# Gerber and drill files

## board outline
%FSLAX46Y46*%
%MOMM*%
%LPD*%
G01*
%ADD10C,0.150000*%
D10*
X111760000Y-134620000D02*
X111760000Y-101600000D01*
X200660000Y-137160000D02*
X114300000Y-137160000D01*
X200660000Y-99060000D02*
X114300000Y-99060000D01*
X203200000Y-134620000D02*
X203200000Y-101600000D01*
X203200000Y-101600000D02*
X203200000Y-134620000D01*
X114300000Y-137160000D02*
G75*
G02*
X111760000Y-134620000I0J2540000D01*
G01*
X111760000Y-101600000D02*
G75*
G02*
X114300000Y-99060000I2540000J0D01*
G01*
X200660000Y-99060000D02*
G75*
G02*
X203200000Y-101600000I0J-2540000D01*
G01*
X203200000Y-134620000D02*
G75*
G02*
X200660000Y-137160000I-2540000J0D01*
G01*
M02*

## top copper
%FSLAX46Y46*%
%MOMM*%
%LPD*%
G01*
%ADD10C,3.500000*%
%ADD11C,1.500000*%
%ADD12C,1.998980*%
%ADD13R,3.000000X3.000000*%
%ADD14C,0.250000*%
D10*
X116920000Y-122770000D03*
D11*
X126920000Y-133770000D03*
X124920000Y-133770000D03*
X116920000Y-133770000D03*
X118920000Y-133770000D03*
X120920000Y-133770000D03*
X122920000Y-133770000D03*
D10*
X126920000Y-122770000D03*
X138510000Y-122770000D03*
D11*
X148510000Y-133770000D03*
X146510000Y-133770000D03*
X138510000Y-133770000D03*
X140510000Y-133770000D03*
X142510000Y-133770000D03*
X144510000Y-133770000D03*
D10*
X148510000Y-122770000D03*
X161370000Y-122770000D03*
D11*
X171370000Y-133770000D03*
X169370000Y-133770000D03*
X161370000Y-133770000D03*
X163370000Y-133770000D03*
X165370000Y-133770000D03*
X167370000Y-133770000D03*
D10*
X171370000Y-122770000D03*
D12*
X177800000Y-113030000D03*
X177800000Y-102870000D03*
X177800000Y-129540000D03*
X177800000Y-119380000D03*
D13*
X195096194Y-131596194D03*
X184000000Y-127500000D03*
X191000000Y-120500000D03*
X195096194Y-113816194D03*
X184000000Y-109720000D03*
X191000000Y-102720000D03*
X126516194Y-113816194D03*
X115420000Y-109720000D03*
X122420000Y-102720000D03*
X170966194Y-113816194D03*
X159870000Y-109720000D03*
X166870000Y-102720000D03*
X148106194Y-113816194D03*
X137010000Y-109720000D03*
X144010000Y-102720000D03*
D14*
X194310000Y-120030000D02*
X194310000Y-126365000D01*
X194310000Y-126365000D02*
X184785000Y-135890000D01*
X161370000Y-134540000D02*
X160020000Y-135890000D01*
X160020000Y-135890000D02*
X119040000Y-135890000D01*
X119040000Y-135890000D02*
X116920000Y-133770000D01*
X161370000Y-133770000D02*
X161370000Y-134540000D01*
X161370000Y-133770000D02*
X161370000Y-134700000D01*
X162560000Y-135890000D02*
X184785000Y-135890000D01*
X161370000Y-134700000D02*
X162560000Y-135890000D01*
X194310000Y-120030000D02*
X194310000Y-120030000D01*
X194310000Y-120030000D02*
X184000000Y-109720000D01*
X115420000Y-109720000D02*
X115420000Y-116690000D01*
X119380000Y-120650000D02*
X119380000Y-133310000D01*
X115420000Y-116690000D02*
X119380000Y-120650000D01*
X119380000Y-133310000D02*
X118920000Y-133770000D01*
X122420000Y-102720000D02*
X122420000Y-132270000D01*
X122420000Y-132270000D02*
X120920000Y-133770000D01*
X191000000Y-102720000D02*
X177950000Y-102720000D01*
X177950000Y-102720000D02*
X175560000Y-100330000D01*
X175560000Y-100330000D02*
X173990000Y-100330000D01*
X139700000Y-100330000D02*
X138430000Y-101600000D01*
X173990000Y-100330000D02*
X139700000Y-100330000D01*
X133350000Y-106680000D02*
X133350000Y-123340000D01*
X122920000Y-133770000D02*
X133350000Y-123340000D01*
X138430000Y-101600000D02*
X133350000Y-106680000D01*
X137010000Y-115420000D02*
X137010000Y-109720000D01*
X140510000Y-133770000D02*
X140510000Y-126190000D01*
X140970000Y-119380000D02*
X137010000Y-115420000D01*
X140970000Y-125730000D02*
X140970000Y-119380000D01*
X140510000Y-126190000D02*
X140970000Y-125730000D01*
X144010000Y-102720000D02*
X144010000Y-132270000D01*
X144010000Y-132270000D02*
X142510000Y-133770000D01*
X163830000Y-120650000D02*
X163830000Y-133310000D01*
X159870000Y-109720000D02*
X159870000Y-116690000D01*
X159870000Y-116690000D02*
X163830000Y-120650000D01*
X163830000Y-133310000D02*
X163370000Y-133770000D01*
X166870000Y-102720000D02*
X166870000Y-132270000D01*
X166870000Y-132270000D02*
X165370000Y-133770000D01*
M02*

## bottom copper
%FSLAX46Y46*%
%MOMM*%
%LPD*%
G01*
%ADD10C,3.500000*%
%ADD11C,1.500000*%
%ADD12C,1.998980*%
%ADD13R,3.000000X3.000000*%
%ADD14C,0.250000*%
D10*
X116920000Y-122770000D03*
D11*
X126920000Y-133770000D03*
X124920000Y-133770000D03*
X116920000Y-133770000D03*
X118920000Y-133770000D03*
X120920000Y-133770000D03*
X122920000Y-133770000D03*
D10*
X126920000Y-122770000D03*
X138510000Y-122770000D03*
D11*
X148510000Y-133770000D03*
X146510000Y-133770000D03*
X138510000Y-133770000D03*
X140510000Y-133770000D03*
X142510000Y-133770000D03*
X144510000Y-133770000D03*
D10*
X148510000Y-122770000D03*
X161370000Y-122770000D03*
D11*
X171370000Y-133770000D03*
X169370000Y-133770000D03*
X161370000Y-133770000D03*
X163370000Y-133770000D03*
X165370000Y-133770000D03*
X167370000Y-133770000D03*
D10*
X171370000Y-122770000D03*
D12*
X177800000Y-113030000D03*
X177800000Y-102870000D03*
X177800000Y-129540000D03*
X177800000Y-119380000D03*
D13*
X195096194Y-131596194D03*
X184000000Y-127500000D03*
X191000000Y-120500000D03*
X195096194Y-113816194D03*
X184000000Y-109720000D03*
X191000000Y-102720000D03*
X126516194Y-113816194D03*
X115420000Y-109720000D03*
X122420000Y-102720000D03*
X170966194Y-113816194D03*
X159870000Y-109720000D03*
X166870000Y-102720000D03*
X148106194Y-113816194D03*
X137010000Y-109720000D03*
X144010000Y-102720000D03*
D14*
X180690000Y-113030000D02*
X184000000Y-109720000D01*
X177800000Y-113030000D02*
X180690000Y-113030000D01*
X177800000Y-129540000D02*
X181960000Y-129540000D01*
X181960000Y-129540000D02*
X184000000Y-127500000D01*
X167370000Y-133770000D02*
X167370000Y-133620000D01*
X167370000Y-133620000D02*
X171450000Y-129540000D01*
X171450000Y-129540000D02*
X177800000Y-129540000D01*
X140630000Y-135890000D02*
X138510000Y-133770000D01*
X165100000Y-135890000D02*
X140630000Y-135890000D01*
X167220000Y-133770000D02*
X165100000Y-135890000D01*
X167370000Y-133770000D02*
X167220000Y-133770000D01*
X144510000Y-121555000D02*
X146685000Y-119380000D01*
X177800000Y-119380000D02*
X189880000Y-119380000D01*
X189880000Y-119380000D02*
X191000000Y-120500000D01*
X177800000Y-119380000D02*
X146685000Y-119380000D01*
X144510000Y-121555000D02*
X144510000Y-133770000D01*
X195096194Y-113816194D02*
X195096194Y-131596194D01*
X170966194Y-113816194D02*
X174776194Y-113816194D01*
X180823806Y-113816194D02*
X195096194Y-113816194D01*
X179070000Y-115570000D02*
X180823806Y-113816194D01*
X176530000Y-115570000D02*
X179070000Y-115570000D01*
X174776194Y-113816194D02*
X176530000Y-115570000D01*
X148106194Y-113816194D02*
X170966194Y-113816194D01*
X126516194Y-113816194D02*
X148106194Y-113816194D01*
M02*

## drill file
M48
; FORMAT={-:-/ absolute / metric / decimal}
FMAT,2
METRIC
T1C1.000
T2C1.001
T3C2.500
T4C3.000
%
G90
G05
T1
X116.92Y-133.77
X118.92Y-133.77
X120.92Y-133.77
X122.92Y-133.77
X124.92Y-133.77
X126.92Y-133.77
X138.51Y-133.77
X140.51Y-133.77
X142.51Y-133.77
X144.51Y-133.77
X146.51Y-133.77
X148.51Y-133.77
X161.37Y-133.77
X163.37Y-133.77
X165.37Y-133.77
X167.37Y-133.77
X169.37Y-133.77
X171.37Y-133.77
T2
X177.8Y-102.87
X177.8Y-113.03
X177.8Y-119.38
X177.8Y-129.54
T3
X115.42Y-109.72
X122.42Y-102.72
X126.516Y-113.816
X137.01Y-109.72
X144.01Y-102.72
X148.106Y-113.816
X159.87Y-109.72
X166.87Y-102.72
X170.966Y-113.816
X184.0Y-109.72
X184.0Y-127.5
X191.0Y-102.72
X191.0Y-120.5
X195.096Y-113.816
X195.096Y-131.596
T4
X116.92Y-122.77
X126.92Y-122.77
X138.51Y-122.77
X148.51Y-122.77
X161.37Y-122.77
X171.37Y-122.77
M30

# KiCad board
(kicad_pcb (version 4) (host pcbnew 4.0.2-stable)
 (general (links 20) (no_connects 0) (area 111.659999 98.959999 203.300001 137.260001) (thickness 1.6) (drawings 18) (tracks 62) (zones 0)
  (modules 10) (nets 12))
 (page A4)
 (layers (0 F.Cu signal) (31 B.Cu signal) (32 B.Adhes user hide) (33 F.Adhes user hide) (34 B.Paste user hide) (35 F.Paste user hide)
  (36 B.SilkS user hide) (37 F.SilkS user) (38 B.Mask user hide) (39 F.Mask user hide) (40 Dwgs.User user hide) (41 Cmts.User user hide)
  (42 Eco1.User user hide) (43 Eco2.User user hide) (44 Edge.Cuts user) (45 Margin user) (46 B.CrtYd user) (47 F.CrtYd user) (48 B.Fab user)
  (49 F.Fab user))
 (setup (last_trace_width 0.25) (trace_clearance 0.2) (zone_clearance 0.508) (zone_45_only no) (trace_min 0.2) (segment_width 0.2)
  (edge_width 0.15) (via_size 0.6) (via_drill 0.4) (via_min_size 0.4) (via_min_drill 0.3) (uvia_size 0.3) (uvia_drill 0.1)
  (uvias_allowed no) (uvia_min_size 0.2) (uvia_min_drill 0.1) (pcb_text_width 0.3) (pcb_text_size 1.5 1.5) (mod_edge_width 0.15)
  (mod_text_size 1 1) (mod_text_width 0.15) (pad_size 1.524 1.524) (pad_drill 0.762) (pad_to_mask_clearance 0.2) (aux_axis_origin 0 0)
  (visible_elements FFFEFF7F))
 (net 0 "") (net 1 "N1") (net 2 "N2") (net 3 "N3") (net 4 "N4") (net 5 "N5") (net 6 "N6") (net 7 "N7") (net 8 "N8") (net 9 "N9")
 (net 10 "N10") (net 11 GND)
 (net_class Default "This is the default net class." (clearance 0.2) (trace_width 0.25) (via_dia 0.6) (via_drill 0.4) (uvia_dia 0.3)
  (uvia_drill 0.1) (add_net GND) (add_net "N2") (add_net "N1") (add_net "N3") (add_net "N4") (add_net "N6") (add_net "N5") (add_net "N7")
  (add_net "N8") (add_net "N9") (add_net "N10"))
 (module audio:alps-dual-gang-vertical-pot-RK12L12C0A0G (layer F.Cu) (at 121.92 128.27)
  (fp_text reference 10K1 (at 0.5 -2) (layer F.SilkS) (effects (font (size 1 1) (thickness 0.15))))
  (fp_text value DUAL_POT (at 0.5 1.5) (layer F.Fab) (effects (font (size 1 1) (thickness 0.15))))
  (pad b thru_hole circle (at -5 -5.5) (size 3.5 3.5) (drill 3) (layers *.Cu *.Mask F.SilkS))
  (pad 3 thru_hole circle (at 5 5.5) (size 1.5 1.5) (drill 1) (layers *.Cu *.Mask F.SilkS))
  (pad 6 thru_hole circle (at 3 5.5) (size 1.5 1.5) (drill 1) (layers *.Cu *.Mask F.SilkS))
  (pad 2 thru_hole circle (at -5 5.5) (size 1.5 1.5) (drill 1) (layers *.Cu *.Mask F.SilkS) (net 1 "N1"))
  (pad 1 thru_hole circle (at -3 5.5) (size 1.5 1.5) (drill 1) (layers *.Cu *.Mask F.SilkS) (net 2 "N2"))
  (pad 4 thru_hole circle (at -1 5.5) (size 1.5 1.5) (drill 1) (layers *.Cu *.Mask F.SilkS) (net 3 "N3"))
  (pad 5 thru_hole circle (at 1 5.5) (size 1.5 1.5) (drill 1) (layers *.Cu *.Mask F.SilkS) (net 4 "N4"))
  (pad a thru_hole circle (at 5 -5.5) (size 3.5 3.5) (drill 3) (layers *.Cu *.Mask F.SilkS)))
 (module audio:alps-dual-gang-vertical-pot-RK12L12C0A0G (layer F.Cu) (at 143.51 128.27)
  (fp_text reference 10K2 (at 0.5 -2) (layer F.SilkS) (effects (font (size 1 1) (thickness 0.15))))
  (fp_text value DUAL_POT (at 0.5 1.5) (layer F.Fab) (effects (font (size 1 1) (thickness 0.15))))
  (pad b thru_hole circle (at -5 -5.5) (size 3.5 3.5) (drill 3) (layers *.Cu *.Mask F.SilkS))
  (pad 3 thru_hole circle (at 5 5.5) (size 1.5 1.5) (drill 1) (layers *.Cu *.Mask F.SilkS))
  (pad 6 thru_hole circle (at 3 5.5) (size 1.5 1.5) (drill 1) (layers *.Cu *.Mask F.SilkS))
  (pad 2 thru_hole circle (at -5 5.5) (size 1.5 1.5) (drill 1) (layers *.Cu *.Mask F.SilkS) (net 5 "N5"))
  (pad 1 thru_hole circle (at -3 5.5) (size 1.5 1.5) (drill 1) (layers *.Cu *.Mask F.SilkS) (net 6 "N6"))
  (pad 4 thru_hole circle (at -1 5.5) (size 1.5 1.5) (drill 1) (layers *.Cu *.Mask F.SilkS) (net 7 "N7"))
  (pad 5 thru_hole circle (at 1 5.5) (size 1.5 1.5) (drill 1) (layers *.Cu *.Mask F.SilkS) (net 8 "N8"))
  (pad a thru_hole circle (at 5 -5.5) (size 3.5 3.5) (drill 3) (layers *.Cu *.Mask F.SilkS)))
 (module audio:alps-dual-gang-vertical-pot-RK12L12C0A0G (layer F.Cu) (at 166.37 128.27)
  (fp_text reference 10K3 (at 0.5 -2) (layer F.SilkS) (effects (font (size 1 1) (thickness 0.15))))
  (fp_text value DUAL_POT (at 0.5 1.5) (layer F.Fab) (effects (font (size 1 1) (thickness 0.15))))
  (pad b thru_hole circle (at -5 -5.5) (size 3.5 3.5) (drill 3) (layers *.Cu *.Mask F.SilkS))
  (pad 3 thru_hole circle (at 5 5.5) (size 1.5 1.5) (drill 1) (layers *.Cu *.Mask F.SilkS))
  (pad 6 thru_hole circle (at 3 5.5) (size 1.5 1.5) (drill 1) (layers *.Cu *.Mask F.SilkS))
  (pad 2 thru_hole circle (at -5 5.5) (size 1.5 1.5) (drill 1) (layers *.Cu *.Mask F.SilkS) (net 1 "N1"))
  (pad 1 thru_hole circle (at -3 5.5) (size 1.5 1.5) (drill 1) (layers *.Cu *.Mask F.SilkS) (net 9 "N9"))
  (pad 4 thru_hole circle (at -1 5.5) (size 1.5 1.5) (drill 1) (layers *.Cu *.Mask F.SilkS) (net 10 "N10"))
  (pad 5 thru_hole circle (at 1 5.5) (size 1.5 1.5) (drill 1) (layers *.Cu *.Mask F.SilkS) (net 5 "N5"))
  (pad a thru_hole circle (at 5 -5.5) (size 3.5 3.5) (drill 3) (layers *.Cu *.Mask F.SilkS)))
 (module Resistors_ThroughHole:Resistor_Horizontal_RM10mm (layer F.Cu) (at 177.8 113.03 90)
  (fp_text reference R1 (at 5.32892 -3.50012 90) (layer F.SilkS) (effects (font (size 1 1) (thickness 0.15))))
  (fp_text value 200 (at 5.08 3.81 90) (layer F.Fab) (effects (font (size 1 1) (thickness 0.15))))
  (pad 1 thru_hole circle (at 0 0 90) (size 1.99898 1.99898) (drill 1.00076) (layers *.Cu *.SilkS *.Mask) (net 1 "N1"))
  (pad 2 thru_hole circle (at 10.16 0 90) (size 1.99898 1.99898) (drill 1.00076) (layers *.Cu *.SilkS *.Mask) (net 4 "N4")))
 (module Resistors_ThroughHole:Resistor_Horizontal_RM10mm (layer F.Cu) (at 177.8 129.54 90)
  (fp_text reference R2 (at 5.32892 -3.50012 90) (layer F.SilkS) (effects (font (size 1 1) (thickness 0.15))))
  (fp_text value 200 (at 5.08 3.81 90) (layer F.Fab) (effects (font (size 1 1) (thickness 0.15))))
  (pad 1 thru_hole circle (at 0 0 90) (size 1.99898 1.99898) (drill 1.00076) (layers *.Cu *.SilkS *.Mask) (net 5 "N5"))
  (pad 2 thru_hole circle (at 10.16 0 90) (size 1.99898 1.99898) (drill 1.00076) (layers *.Cu *.SilkS *.Mask) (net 8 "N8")))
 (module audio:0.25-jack (layer F.Cu) (at 190.5 127)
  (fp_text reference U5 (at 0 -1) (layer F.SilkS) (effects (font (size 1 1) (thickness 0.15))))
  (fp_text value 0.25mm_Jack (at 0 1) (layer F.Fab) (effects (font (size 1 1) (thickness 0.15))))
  (pad 3 thru_hole rect (at 4.596194 4.596194) (size 3 3) (drill oval 2.5) (layers *.Cu *.Mask F.SilkS) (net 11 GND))
  (pad 1 thru_hole rect (at -6.5 0.5) (size 3 3) (drill oval 2.5) (layers *.Cu *.Mask F.SilkS) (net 5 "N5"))
  (pad 2 thru_hole rect (at 0.5 -6.5 90) (size 3 3) (drill oval 2.5) (layers *.Cu *.Mask F.SilkS) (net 8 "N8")))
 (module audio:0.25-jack (layer F.Cu) (at 190.5 109.22)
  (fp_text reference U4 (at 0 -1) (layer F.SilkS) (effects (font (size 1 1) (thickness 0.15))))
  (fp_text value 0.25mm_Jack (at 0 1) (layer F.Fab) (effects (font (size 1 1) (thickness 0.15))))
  (pad 3 thru_hole rect (at 4.596194 4.596194) (size 3 3) (drill oval 2.5) (layers *.Cu *.Mask F.SilkS) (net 11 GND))
  (pad 1 thru_hole rect (at -6.5 0.5) (size 3 3) (drill oval 2.5) (layers *.Cu *.Mask F.SilkS) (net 1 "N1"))
  (pad 2 thru_hole rect (at 0.5 -6.5 90) (size 3 3) (drill oval 2.5) (layers *.Cu *.Mask F.SilkS) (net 4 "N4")))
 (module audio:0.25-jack (layer F.Cu) (at 121.92 109.22)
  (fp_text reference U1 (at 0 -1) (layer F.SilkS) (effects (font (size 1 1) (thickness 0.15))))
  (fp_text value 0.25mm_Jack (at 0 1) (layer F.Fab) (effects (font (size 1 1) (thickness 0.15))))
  (pad 3 thru_hole rect (at 4.596194 4.596194) (size 3 3) (drill oval 2.5) (layers *.Cu *.Mask F.SilkS) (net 11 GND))
  (pad 1 thru_hole rect (at -6.5 0.5) (size 3 3) (drill oval 2.5) (layers *.Cu *.Mask F.SilkS) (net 2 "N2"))
  (pad 2 thru_hole rect (at 0.5 -6.5 90) (size 3 3) (drill oval 2.5) (layers *.Cu *.Mask F.SilkS) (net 3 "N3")))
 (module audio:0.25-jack (layer F.Cu) (at 166.37 109.22)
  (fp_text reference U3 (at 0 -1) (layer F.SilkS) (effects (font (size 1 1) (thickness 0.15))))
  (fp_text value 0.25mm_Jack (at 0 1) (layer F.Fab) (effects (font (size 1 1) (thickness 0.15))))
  (pad 3 thru_hole rect (at 4.596194 4.596194) (size 3 3) (drill oval 2.5) (layers *.Cu *.Mask F.SilkS) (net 11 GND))
  (pad 1 thru_hole rect (at -6.5 0.5) (size 3 3) (drill oval 2.5) (layers *.Cu *.Mask F.SilkS) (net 9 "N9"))
  (pad 2 thru_hole rect (at 0.5 -6.5 90) (size 3 3) (drill oval 2.5) (layers *.Cu *.Mask F.SilkS) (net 10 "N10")))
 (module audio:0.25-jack (layer F.Cu) (at 143.51 109.22)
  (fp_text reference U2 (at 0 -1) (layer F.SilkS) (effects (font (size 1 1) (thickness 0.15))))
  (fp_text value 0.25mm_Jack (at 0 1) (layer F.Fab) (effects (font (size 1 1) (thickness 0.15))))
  (pad 3 thru_hole rect (at 4.596194 4.596194) (size 3 3) (drill oval 2.5) (layers *.Cu *.Mask F.SilkS) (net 11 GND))
  (pad 1 thru_hole rect (at -6.5 0.5) (size 3 3) (drill oval 2.5) (layers *.Cu *.Mask F.SilkS) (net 6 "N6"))
  (pad 2 thru_hole rect (at 0.5 -6.5 90) (size 3 3) (drill oval 2.5) (layers *.Cu *.Mask F.SilkS) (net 7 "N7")))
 (gr_line (start 111.76 134.62) (end 111.76 101.6) (angle 90) (layer Edge.Cuts) (width 0.15))
 (gr_line (start 200.66 137.16) (end 114.3 137.16) (angle 90) (layer Edge.Cuts) (width 0.15))
 (gr_line (start 200.66 99.06) (end 114.3 99.06) (angle 90) (layer Edge.Cuts) (width 0.15))
 (gr_line (start 203.2 134.62) (end 203.2 101.6) (angle 90) (layer Edge.Cuts) (width 0.15))
 (gr_line (start 203.2 101.6) (end 203.2 134.62) (angle 90) (layer Edge.Cuts) (width 0.15))
 (gr_arc (start 114.3 134.62) (end 114.3 137.16) (angle 90) (layer Edge.Cuts) (width 0.15))
 (gr_arc (start 114.3 101.6) (end 111.76 101.6) (angle 90) (layer Edge.Cuts) (width 0.15))
 (gr_arc (start 200.66 101.6) (end 200.66 99.06) (angle 90) (layer Edge.Cuts) (width 0.15))
 (gr_arc (start 200.66 134.62) (end 203.2 134.62) (angle 90) (layer Edge.Cuts) (width 0.15))
 (segment (start 194.31 120.03) (end 194.31 126.365) (width 0.25) (layer F.Cu) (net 1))
 (segment (start 194.31 126.365) (end 184.785 135.89) (width 0.25) (layer F.Cu) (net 1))
 (segment (start 161.37 134.54) (end 160.02 135.89) (width 0.25) (layer F.Cu) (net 1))
 (segment (start 160.02 135.89) (end 119.04 135.89) (width 0.25) (layer F.Cu) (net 1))
 (segment (start 119.04 135.89) (end 116.92 133.77) (width 0.25) (layer F.Cu) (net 1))
 (segment (start 161.37 133.77) (end 161.37 134.54) (width 0.25) (layer F.Cu) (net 1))
 (segment (start 161.37 133.77) (end 161.37 134.7) (width 0.25) (layer F.Cu) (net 1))
 (segment (start 162.56 135.89) (end 184.785 135.89) (width 0.25) (layer F.Cu) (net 1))
 (segment (start 161.37 134.7) (end 162.56 135.89) (width 0.25) (layer F.Cu) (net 1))
 (segment (start 194.31 120.03) (end 194.31 120.03) (width 0.25) (layer F.Cu) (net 1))
 (segment (start 194.31 120.03) (end 184 109.72) (width 0.25) (layer F.Cu) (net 1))
 (segment (start 180.69 113.03) (end 184 109.72) (width 0.25) (layer B.Cu) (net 1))
 (segment (start 177.8 113.03) (end 180.69 113.03) (width 0.25) (layer B.Cu) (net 1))
 (segment (start 115.42 109.72) (end 115.42 116.69) (width 0.25) (layer F.Cu) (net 2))
 (segment (start 119.38 120.65) (end 119.38 133.31) (width 0.25) (layer F.Cu) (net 2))
 (segment (start 115.42 116.69) (end 119.38 120.65) (width 0.25) (layer F.Cu) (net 2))
 (segment (start 119.38 133.31) (end 118.92 133.77) (width 0.25) (layer F.Cu) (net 2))
 (segment (start 122.42 102.72) (end 122.42 132.27) (width 0.25) (layer F.Cu) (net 3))
 (segment (start 122.42 132.27) (end 120.92 133.77) (width 0.25) (layer F.Cu) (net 3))
 (segment (start 191 102.72) (end 177.95 102.72) (width 0.25) (layer F.Cu) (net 4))
 (segment (start 177.95 102.72) (end 175.56 100.33) (width 0.25) (layer F.Cu) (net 4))
 (segment (start 175.56 100.33) (end 173.99 100.33) (width 0.25) (layer F.Cu) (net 4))
 (segment (start 139.7 100.33) (end 138.43 101.6) (width 0.25) (layer F.Cu) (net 4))
 (segment (start 173.99 100.33) (end 139.7 100.33) (width 0.25) (layer F.Cu) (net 4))
 (segment (start 133.35 106.68) (end 133.35 123.34) (width 0.25) (layer F.Cu) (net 4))
 (segment (start 122.92 133.77) (end 133.35 123.34) (width 0.25) (layer F.Cu) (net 4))
 (segment (start 138.43 101.6) (end 133.35 106.68) (width 0.25) (layer F.Cu) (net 4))
 (segment (start 177.8 129.54) (end 181.96 129.54) (width 0.25) (layer B.Cu) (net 5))
 (segment (start 181.96 129.54) (end 184 127.5) (width 0.25) (layer B.Cu) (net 5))
 (segment (start 167.37 133.77) (end 167.37 133.62) (width 0.25) (layer B.Cu) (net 5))
 (segment (start 167.37 133.62) (end 171.45 129.54) (width 0.25) (layer B.Cu) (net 5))
 (segment (start 171.45 129.54) (end 177.8 129.54) (width 0.25) (layer B.Cu) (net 5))
 (segment (start 140.63 135.89) (end 138.51 133.77) (width 0.25) (layer B.Cu) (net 5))
 (segment (start 165.1 135.89) (end 140.63 135.89) (width 0.25) (layer B.Cu) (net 5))
 (segment (start 167.22 133.77) (end 165.1 135.89) (width 0.25) (layer B.Cu) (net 5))
 (segment (start 167.37 133.77) (end 167.22 133.77) (width 0.25) (layer B.Cu) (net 5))
 (segment (start 137.01 115.42) (end 137.01 109.72) (width 0.25) (layer F.Cu) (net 6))
 (segment (start 140.51 133.77) (end 140.51 126.19) (width 0.25) (layer F.Cu) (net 6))
 (segment (start 140.97 119.38) (end 137.01 115.42) (width 0.25) (layer F.Cu) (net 6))
 (segment (start 140.97 125.73) (end 140.97 119.38) (width 0.25) (layer F.Cu) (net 6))
 (segment (start 140.51 126.19) (end 140.97 125.73) (width 0.25) (layer F.Cu) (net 6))
 (segment (start 144.01 102.72) (end 144.01 132.27) (width 0.25) (layer F.Cu) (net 7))
 (segment (start 144.01 132.27) (end 142.51 133.77) (width 0.25) (layer F.Cu) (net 7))
 (segment (start 144.51 121.555) (end 146.685 119.38) (width 0.25) (layer B.Cu) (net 8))
 (segment (start 177.8 119.38) (end 189.88 119.38) (width 0.25) (layer B.Cu) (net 8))
 (segment (start 189.88 119.38) (end 191 120.5) (width 0.25) (layer B.Cu) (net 8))
 (segment (start 177.8 119.38) (end 146.685 119.38) (width 0.25) (layer B.Cu) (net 8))
 (segment (start 144.51 121.555) (end 144.51 133.77) (width 0.25) (layer B.Cu) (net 8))
 (segment (start 163.83 120.65) (end 163.83 133.31) (width 0.25) (layer F.Cu) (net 9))
 (segment (start 159.87 109.72) (end 159.87 116.69) (width 0.25) (layer F.Cu) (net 9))
 (segment (start 159.87 116.69) (end 163.83 120.65) (width 0.25) (layer F.Cu) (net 9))
 (segment (start 163.83 133.31) (end 163.37 133.77) (width 0.25) (layer F.Cu) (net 9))
 (segment (start 166.87 102.72) (end 166.87 132.27) (width 0.25) (layer F.Cu) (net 10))
 (segment (start 166.87 132.27) (end 165.37 133.77) (width 0.25) (layer F.Cu) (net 10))
 (segment (start 195.096194 113.816194) (end 195.096194 131.596194) (width 0.25) (layer B.Cu) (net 11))
 (segment (start 170.966194 113.816194) (end 174.776194 113.816194) (width 0.25) (layer B.Cu) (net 11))
 (segment (start 180.823806 113.816194) (end 195.096194 113.816194) (width 0.25) (layer B.Cu) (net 11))
 (segment (start 179.07 115.57) (end 180.823806 113.816194) (width 0.25) (layer B.Cu) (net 11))
 (segment (start 176.53 115.57) (end 179.07 115.57) (width 0.25) (layer B.Cu) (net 11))
 (segment (start 174.776194 113.816194) (end 176.53 115.57) (width 0.25) (layer B.Cu) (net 11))
 (segment (start 148.106194 113.816194) (end 170.966194 113.816194) (width 0.25) (layer B.Cu) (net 11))
 (segment (start 126.516194 113.816194) (end 148.106194 113.816194) (width 0.25) (layer B.Cu) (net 11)))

